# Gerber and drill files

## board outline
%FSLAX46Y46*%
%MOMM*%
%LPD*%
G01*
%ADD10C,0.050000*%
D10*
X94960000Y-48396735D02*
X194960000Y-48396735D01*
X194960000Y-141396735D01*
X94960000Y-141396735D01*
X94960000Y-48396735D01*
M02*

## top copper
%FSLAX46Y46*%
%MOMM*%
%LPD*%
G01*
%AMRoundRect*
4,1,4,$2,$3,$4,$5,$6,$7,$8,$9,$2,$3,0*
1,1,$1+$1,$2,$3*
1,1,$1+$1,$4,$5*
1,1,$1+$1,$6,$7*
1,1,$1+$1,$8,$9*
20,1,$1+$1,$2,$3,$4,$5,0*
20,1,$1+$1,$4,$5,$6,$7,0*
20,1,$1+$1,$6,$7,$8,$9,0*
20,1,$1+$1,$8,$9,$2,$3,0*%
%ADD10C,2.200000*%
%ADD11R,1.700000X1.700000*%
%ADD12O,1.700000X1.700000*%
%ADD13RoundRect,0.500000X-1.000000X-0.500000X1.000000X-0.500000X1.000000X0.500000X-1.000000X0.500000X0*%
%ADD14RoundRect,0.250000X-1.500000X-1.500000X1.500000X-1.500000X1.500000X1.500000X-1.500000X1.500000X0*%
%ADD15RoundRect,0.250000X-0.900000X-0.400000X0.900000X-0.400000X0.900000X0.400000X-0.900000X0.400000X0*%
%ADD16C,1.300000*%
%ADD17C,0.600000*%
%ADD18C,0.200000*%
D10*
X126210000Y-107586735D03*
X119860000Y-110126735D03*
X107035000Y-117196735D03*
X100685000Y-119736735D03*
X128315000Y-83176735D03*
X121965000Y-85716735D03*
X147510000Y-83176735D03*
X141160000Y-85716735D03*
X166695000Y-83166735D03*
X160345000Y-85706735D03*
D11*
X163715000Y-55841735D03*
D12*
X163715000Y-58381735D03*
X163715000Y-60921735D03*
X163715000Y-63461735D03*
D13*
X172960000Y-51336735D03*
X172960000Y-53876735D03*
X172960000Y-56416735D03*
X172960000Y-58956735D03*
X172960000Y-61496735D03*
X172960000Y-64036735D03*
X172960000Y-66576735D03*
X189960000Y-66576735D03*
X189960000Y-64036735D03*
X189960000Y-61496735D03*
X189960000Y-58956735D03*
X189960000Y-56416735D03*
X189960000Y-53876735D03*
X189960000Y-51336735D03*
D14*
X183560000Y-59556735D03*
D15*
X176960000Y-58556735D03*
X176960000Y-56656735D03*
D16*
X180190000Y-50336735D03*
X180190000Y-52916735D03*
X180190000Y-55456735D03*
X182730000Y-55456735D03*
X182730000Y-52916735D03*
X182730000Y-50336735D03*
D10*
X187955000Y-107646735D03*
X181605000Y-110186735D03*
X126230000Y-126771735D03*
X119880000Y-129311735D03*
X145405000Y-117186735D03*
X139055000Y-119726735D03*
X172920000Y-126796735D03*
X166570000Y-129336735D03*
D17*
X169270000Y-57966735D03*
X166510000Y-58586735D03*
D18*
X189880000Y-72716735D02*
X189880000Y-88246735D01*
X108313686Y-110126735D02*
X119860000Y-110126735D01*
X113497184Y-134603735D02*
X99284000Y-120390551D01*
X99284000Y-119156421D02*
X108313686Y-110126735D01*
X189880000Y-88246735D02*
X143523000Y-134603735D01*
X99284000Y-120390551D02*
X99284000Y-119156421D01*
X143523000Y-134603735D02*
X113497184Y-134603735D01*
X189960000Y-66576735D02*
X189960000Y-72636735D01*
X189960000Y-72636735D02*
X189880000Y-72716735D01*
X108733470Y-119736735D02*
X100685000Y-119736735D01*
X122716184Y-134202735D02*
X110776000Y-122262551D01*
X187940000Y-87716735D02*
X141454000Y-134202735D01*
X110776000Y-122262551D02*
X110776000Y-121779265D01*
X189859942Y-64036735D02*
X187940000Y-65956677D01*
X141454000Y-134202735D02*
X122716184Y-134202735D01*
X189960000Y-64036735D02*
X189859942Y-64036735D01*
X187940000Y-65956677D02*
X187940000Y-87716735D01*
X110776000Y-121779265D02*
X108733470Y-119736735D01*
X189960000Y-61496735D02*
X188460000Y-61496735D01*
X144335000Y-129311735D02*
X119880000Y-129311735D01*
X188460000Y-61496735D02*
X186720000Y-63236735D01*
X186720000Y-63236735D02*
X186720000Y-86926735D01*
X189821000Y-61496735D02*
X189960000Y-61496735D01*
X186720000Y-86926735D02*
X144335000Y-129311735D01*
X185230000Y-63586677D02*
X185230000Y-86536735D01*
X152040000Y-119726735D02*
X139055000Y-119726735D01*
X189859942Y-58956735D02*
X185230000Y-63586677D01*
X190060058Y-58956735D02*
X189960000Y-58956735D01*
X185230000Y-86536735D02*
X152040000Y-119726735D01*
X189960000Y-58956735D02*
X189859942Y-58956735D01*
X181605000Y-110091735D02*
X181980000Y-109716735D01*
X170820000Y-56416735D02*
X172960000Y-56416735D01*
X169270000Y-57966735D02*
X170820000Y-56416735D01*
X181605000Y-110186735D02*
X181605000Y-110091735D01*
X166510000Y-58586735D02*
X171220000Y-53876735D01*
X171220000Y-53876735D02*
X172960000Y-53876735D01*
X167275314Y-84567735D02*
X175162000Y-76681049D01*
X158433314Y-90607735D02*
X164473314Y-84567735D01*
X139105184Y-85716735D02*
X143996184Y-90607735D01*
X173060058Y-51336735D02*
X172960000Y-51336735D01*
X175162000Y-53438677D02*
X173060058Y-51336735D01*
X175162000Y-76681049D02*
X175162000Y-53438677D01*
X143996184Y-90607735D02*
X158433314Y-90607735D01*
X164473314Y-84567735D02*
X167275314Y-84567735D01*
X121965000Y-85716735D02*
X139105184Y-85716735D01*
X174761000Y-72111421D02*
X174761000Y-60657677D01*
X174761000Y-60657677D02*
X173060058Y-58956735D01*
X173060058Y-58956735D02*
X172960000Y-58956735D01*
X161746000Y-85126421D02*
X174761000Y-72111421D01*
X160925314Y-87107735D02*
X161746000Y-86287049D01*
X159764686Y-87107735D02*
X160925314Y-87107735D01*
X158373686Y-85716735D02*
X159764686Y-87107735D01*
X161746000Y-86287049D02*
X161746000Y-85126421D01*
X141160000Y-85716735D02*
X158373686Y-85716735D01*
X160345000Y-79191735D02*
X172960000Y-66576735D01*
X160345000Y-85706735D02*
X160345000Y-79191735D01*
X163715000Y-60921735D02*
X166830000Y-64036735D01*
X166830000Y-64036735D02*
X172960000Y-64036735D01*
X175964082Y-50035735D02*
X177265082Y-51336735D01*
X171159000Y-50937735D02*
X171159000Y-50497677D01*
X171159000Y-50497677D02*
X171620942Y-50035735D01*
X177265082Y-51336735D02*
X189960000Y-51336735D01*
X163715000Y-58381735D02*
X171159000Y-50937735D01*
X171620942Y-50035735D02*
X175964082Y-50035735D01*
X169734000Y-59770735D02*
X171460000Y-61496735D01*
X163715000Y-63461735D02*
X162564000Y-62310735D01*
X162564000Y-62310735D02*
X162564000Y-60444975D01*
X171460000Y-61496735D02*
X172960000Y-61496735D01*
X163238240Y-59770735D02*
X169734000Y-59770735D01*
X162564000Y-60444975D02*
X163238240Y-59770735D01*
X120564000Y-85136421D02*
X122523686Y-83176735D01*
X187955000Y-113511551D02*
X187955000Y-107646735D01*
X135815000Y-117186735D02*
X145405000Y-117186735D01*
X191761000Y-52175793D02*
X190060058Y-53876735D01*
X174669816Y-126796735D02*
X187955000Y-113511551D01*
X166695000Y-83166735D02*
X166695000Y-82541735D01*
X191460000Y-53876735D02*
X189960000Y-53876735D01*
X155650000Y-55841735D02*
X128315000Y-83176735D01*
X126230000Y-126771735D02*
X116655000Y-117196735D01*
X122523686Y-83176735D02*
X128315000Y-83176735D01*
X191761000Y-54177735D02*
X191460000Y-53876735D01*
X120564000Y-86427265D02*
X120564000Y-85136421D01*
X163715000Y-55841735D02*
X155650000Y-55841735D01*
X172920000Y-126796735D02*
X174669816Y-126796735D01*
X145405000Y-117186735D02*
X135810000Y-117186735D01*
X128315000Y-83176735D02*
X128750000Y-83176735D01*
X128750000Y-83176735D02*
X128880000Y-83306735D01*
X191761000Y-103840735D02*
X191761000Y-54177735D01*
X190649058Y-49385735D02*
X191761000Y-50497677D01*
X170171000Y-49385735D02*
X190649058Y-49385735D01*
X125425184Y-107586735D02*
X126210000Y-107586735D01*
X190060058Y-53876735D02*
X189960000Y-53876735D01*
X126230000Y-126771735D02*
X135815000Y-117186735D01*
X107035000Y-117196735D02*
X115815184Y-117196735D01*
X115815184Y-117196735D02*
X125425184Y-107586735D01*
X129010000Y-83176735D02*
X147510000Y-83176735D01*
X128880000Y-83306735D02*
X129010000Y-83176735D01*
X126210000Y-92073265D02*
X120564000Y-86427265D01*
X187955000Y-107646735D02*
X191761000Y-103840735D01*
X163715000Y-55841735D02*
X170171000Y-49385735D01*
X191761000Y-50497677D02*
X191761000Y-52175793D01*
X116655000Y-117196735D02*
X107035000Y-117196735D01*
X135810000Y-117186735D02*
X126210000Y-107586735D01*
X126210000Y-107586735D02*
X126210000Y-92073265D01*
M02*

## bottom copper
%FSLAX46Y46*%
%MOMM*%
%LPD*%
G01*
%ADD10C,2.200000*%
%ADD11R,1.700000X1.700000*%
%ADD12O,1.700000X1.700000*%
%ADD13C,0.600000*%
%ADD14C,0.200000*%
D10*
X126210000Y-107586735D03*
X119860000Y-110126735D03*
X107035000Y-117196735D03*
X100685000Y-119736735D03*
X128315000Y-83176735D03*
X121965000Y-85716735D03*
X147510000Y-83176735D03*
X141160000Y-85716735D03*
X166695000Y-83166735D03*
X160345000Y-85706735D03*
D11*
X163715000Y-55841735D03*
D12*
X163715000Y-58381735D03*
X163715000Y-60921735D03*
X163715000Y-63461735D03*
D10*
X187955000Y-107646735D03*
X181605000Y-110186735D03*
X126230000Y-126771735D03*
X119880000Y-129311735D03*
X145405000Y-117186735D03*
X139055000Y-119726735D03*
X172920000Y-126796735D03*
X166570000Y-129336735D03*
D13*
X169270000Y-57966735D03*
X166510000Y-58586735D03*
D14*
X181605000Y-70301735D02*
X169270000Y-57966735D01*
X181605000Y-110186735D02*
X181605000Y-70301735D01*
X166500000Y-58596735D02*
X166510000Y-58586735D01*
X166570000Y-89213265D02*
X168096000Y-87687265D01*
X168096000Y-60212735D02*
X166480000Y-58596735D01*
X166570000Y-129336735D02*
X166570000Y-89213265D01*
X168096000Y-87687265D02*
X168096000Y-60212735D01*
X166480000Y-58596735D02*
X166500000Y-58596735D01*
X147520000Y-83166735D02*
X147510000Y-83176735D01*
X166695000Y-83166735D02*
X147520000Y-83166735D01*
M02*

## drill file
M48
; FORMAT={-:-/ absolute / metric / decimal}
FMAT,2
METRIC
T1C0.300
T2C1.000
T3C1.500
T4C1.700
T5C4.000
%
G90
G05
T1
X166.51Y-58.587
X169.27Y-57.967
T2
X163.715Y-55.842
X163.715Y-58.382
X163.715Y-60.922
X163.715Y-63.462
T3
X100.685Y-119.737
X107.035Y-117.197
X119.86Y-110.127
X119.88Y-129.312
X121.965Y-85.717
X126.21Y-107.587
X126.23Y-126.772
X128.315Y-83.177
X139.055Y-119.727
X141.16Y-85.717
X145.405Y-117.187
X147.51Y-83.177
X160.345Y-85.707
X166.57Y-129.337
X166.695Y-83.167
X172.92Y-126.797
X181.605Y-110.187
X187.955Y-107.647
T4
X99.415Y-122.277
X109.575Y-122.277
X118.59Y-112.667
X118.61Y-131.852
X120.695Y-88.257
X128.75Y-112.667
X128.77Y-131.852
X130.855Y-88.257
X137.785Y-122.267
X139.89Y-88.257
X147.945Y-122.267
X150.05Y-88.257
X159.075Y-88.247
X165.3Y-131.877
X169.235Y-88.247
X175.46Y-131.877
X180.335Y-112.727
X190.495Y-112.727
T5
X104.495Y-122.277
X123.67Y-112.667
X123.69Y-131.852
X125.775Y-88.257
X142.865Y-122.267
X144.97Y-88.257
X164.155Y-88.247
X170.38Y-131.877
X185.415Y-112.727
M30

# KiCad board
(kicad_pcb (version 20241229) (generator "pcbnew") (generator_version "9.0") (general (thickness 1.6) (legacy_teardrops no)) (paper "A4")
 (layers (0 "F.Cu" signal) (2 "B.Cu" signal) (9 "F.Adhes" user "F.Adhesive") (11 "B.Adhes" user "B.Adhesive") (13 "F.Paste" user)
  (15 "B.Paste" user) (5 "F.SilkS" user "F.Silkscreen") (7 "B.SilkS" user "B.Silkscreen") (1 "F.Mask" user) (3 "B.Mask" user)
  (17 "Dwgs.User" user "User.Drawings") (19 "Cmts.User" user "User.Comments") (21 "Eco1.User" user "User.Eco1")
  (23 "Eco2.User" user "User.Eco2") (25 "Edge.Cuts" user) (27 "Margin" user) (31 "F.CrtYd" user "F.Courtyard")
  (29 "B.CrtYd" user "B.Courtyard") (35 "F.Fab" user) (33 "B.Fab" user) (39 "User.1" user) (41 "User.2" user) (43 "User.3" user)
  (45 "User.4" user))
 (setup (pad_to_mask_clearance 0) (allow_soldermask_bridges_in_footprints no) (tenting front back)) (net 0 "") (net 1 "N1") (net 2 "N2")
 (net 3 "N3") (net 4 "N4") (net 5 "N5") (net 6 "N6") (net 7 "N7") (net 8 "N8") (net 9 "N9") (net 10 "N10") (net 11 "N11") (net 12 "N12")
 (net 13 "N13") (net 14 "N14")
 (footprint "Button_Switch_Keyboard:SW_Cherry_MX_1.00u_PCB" (layer "F.Cu") (at 126.21 107.586735)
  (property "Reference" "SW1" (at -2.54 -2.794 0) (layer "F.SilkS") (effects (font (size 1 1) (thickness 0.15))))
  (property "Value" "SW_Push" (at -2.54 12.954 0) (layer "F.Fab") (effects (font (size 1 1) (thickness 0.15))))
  (pad "" np_thru_hole circle (at -7.62 5.08) (size 1.7 1.7) (drill 1.7) (layers "*.Cu" "*.Mask"))
  (pad "" np_thru_hole circle (at -2.54 5.08) (size 4 4) (drill 4) (layers "*.Cu" "*.Mask"))
  (pad "" np_thru_hole circle (at 2.54 5.08) (size 1.7 1.7) (drill 1.7) (layers "*.Cu" "*.Mask"))
  (pad "1" thru_hole circle (at 0 0) (size 2.2 2.2) (drill 1.5) (layers "*.Cu" "*.Mask") (remove_unused_layers no) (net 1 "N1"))
  (pad "2" thru_hole circle (at -6.35 2.54) (size 2.2 2.2) (drill 1.5) (layers "*.Cu" "*.Mask") (remove_unused_layers no) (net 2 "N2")))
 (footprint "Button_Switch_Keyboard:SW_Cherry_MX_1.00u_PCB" (layer "F.Cu") (at 107.035 117.196735)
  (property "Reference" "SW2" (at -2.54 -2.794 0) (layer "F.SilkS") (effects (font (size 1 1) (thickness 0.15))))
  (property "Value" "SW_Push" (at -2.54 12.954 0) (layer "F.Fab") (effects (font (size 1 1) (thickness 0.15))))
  (pad "" np_thru_hole circle (at -7.62 5.08) (size 1.7 1.7) (drill 1.7) (layers "*.Cu" "*.Mask"))
  (pad "" np_thru_hole circle (at -2.54 5.08) (size 4 4) (drill 4) (layers "*.Cu" "*.Mask"))
  (pad "" np_thru_hole circle (at 2.54 5.08) (size 1.7 1.7) (drill 1.7) (layers "*.Cu" "*.Mask"))
  (pad "1" thru_hole circle (at 0 0) (size 2.2 2.2) (drill 1.5) (layers "*.Cu" "*.Mask") (remove_unused_layers no) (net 1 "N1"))
  (pad "2" thru_hole circle (at -6.35 2.54) (size 2.2 2.2) (drill 1.5) (layers "*.Cu" "*.Mask") (remove_unused_layers no) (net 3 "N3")))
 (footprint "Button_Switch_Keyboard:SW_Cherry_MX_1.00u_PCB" (layer "F.Cu") (at 128.315 83.176735)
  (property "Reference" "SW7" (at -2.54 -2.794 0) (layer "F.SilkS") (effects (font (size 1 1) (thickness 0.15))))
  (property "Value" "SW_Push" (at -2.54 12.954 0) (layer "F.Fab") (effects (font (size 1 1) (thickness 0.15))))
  (pad "" np_thru_hole circle (at -7.62 5.08) (size 1.7 1.7) (drill 1.7) (layers "*.Cu" "*.Mask"))
  (pad "" np_thru_hole circle (at -2.54 5.08) (size 4 4) (drill 4) (layers "*.Cu" "*.Mask"))
  (pad "" np_thru_hole circle (at 2.54 5.08) (size 1.7 1.7) (drill 1.7) (layers "*.Cu" "*.Mask"))
  (pad "1" thru_hole circle (at 0 0) (size 2.2 2.2) (drill 1.5) (layers "*.Cu" "*.Mask") (remove_unused_layers no) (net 1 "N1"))
  (pad "2" thru_hole circle (at -6.35 2.54) (size 2.2 2.2) (drill 1.5) (layers "*.Cu" "*.Mask") (remove_unused_layers no) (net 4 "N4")))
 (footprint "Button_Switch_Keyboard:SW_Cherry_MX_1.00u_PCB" (layer "F.Cu") (at 147.51 83.176735)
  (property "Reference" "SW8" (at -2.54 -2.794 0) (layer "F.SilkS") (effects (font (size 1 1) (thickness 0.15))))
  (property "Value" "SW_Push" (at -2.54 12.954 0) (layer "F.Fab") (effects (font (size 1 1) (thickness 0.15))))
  (pad "" np_thru_hole circle (at -7.62 5.08) (size 1.7 1.7) (drill 1.7) (layers "*.Cu" "*.Mask"))
  (pad "" np_thru_hole circle (at -2.54 5.08) (size 4 4) (drill 4) (layers "*.Cu" "*.Mask"))
  (pad "" np_thru_hole circle (at 2.54 5.08) (size 1.7 1.7) (drill 1.7) (layers "*.Cu" "*.Mask"))
  (pad "1" thru_hole circle (at 0 0) (size 2.2 2.2) (drill 1.5) (layers "*.Cu" "*.Mask") (remove_unused_layers no) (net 1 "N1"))
  (pad "2" thru_hole circle (at -6.35 2.54) (size 2.2 2.2) (drill 1.5) (layers "*.Cu" "*.Mask") (remove_unused_layers no) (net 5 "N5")))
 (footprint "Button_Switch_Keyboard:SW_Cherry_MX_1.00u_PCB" (layer "F.Cu") (at 166.695 83.166735)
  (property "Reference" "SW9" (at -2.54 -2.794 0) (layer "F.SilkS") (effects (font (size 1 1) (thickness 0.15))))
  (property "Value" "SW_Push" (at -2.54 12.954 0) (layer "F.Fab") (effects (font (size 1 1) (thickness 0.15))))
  (pad "" np_thru_hole circle (at -7.62 5.08) (size 1.7 1.7) (drill 1.7) (layers "*.Cu" "*.Mask"))
  (pad "" np_thru_hole circle (at -2.54 5.08) (size 4 4) (drill 4) (layers "*.Cu" "*.Mask"))
  (pad "" np_thru_hole circle (at 2.54 5.08) (size 1.7 1.7) (drill 1.7) (layers "*.Cu" "*.Mask"))
  (pad "1" thru_hole circle (at 0 0) (size 2.2 2.2) (drill 1.5) (layers "*.Cu" "*.Mask") (remove_unused_layers no) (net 1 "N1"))
  (pad "2" thru_hole circle (at -6.35 2.54) (size 2.2 2.2) (drill 1.5) (layers "*.Cu" "*.Mask") (remove_unused_layers no) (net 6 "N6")))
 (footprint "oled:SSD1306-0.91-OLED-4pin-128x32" (layer "F.Cu") (at 127.215 53.651735)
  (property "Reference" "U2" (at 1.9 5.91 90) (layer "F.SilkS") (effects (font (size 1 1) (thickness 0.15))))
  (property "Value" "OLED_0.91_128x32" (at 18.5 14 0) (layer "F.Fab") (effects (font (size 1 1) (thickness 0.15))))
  (pad "1" thru_hole rect (at 36.5 2.19) (size 1.7 1.7) (drill 1) (layers "*.Cu" "*.Mask") (remove_unused_layers no) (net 1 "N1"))
  (pad "2" thru_hole oval (at 36.5 4.73) (size 1.7 1.7) (drill 1) (layers "*.Cu" "*.Mask") (remove_unused_layers no) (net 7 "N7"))
  (pad "3" thru_hole oval (at 36.5 7.27) (size 1.7 1.7) (drill 1) (layers "*.Cu" "*.Mask") (remove_unused_layers no) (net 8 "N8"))
  (pad "4" thru_hole oval (at 36.5 9.81) (size 1.7 1.7) (drill 1) (layers "*.Cu" "*.Mask") (remove_unused_layers no) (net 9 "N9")))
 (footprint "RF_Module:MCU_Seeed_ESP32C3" (layer "F.Cu") (at 181.46 58.956735)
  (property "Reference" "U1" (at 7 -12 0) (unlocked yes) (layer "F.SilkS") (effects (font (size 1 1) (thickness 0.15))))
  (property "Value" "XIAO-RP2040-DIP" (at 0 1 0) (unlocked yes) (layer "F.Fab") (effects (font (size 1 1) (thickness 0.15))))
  (pad "" smd roundrect (at 1.1 -0.4) (size 1.5 1.5) (layers "F.Paste") (roundrect_rratio 0.1666666667))
  (pad "" smd roundrect (at 1.1 1.6) (size 1.5 1.5) (layers "F.Paste") (roundrect_rratio 0.1666666667))
  (pad "" smd roundrect (at 3.1 -0.4) (size 1.5 1.5) (layers "F.Paste") (roundrect_rratio 0.1666666667))
  (pad "" smd roundrect (at 3.1 1.6) (size 1.5 1.5) (layers "F.Paste") (roundrect_rratio 0.1666666667))
  (pad "1" smd roundrect (at -8.5 -7.62) (size 3 2) (layers "F.Cu" "F.Mask" "F.Paste") (roundrect_rratio 0.25) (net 4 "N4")
   (thermal_bridge_angle 45))
  (pad "2" smd roundrect (at -8.5 -5.08) (size 3 2) (layers "F.Cu" "F.Mask" "F.Paste") (roundrect_rratio 0.25) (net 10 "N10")
   (thermal_bridge_angle 45))
  (pad "3" smd roundrect (at -8.5 -2.54) (size 3 2) (layers "F.Cu" "F.Mask" "F.Paste") (roundrect_rratio 0.25) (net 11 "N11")
   (thermal_bridge_angle 45))
  (pad "4" smd roundrect (at -8.5 0) (size 3 2) (layers "F.Cu" "F.Mask" "F.Paste") (roundrect_rratio 0.25) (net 5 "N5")
   (thermal_bridge_angle 45))
  (pad "5" smd roundrect (at -8.5 2.54) (size 3 2) (layers "F.Cu" "F.Mask" "F.Paste") (roundrect_rratio 0.25) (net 9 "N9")
   (thermal_bridge_angle 45))
  (pad "6" smd roundrect (at -8.5 5.08) (size 3 2) (layers "F.Cu" "F.Mask" "F.Paste") (roundrect_rratio 0.25) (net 8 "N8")
   (thermal_bridge_angle 45))
  (pad "7" smd roundrect (at -8.5 7.62) (size 3 2) (layers "F.Cu" "F.Mask" "F.Paste") (roundrect_rratio 0.25) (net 6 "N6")
   (thermal_bridge_angle 45))
  (pad "8" smd roundrect (at 8.5 7.62) (size 3 2) (layers "F.Cu" "F.Mask" "F.Paste") (roundrect_rratio 0.25) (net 2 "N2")
   (thermal_bridge_angle 45))
  (pad "9" smd roundrect (at 8.5 5.08) (size 3 2) (layers "F.Cu" "F.Mask" "F.Paste") (roundrect_rratio 0.25) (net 3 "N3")
   (thermal_bridge_angle 45))
  (pad "10" smd roundrect (at 8.5 2.54) (size 3 2) (layers "F.Cu" "F.Mask" "F.Paste") (roundrect_rratio 0.25) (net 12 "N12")
   (thermal_bridge_angle 45))
  (pad "11" smd roundrect (at 8.5 0) (size 3 2) (layers "F.Cu" "F.Mask" "F.Paste") (roundrect_rratio 0.25) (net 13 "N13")
   (thermal_bridge_angle 45))
  (pad "12" smd roundrect (at 8.5 -2.54) (size 3 2) (layers "F.Cu" "F.Mask" "F.Paste") (roundrect_rratio 0.25) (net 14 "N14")
   (thermal_bridge_angle 45))
  (pad "13" smd roundrect (at 8.5 -5.08) (size 3 2) (layers "F.Cu" "F.Mask" "F.Paste") (roundrect_rratio 0.25) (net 1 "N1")
   (thermal_bridge_angle 45))
  (pad "14" smd roundrect (at 8.5 -7.62) (size 3 2) (layers "F.Cu" "F.Mask" "F.Paste") (roundrect_rratio 0.25) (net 7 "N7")
   (thermal_bridge_angle 45))
  (pad "15" smd roundrect (at 2.1 0.6) (size 3.5 3.5) (layers "F.Cu" "F.Mask") (roundrect_rratio 0.07142857143))
  (pad "16" smd roundrect (at -4.5 -0.4) (size 2.3 1.3) (layers "F.Cu" "F.Mask" "F.Paste") (roundrect_rratio 0.1923076923))
  (pad "17" smd roundrect (at -4.5 -2.3) (size 2.3 1.3) (layers "F.Cu" "F.Mask" "F.Paste") (roundrect_rratio 0.1923076923))
  (pad "18" smd circle (at -1.27 -8.62) (size 1.3 1.3) (layers "F.Cu" "F.Mask" "F.Paste"))
  (pad "19" smd circle (at -1.27 -6.04) (size 1.3 1.3) (layers "F.Cu" "F.Mask" "F.Paste"))
  (pad "20" smd circle (at -1.27 -3.5) (size 1.3 1.3) (layers "F.Cu" "F.Mask" "F.Paste"))
  (pad "21" smd circle (at 1.27 -3.5) (size 1.3 1.3) (layers "F.Cu" "F.Mask" "F.Paste"))
  (pad "22" smd circle (at 1.27 -6.04) (size 1.3 1.3) (layers "F.Cu" "F.Mask" "F.Paste"))
  (pad "23" smd circle (at 1.27 -8.62) (size 1.3 1.3) (layers "F.Cu" "F.Mask" "F.Paste")))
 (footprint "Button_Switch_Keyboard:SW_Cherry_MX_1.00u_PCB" (layer "F.Cu") (at 187.955 107.646735)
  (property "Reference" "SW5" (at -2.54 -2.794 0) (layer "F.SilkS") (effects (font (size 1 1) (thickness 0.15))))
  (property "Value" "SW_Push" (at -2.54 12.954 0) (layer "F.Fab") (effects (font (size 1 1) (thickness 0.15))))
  (pad "" np_thru_hole circle (at -7.62 5.08) (size 1.7 1.7) (drill 1.7) (layers "*.Cu" "*.Mask"))
  (pad "" np_thru_hole circle (at -2.54 5.08) (size 4 4) (drill 4) (layers "*.Cu" "*.Mask"))
  (pad "" np_thru_hole circle (at 2.54 5.08) (size 1.7 1.7) (drill 1.7) (layers "*.Cu" "*.Mask"))
  (pad "1" thru_hole circle (at 0 0) (size 2.2 2.2) (drill 1.5) (layers "*.Cu" "*.Mask") (remove_unused_layers no) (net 1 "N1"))
  (pad "2" thru_hole circle (at -6.35 2.54) (size 2.2 2.2) (drill 1.5) (layers "*.Cu" "*.Mask") (remove_unused_layers no) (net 11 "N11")))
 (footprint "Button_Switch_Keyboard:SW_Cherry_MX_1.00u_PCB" (layer "F.Cu") (at 126.23 126.771735)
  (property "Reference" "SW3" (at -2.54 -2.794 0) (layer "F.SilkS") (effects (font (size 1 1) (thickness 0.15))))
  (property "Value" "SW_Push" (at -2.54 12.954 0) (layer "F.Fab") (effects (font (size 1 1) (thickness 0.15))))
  (pad "" np_thru_hole circle (at -7.62 5.08) (size 1.7 1.7) (drill 1.7) (layers "*.Cu" "*.Mask"))
  (pad "" np_thru_hole circle (at -2.54 5.08) (size 4 4) (drill 4) (layers "*.Cu" "*.Mask"))
  (pad "" np_thru_hole circle (at 2.54 5.08) (size 1.7 1.7) (drill 1.7) (layers "*.Cu" "*.Mask"))
  (pad "1" thru_hole circle (at 0 0) (size 2.2 2.2) (drill 1.5) (layers "*.Cu" "*.Mask") (remove_unused_layers no) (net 1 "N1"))
  (pad "2" thru_hole circle (at -6.35 2.54) (size 2.2 2.2) (drill 1.5) (layers "*.Cu" "*.Mask") (remove_unused_layers no) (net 12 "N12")))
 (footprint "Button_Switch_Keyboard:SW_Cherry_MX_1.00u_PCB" (layer "F.Cu") (at 145.405 117.186735)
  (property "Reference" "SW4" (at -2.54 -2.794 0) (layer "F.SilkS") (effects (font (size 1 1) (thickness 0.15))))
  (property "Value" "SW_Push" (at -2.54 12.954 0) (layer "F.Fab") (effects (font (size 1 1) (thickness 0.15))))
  (pad "" np_thru_hole circle (at -7.62 5.08) (size 1.7 1.7) (drill 1.7) (layers "*.Cu" "*.Mask"))
  (pad "" np_thru_hole circle (at -2.54 5.08) (size 4 4) (drill 4) (layers "*.Cu" "*.Mask"))
  (pad "" np_thru_hole circle (at 2.54 5.08) (size 1.7 1.7) (drill 1.7) (layers "*.Cu" "*.Mask"))
  (pad "1" thru_hole circle (at 0 0) (size 2.2 2.2) (drill 1.5) (layers "*.Cu" "*.Mask") (remove_unused_layers no) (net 1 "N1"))
  (pad "2" thru_hole circle (at -6.35 2.54) (size 2.2 2.2) (drill 1.5) (layers "*.Cu" "*.Mask") (remove_unused_layers no) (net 13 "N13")))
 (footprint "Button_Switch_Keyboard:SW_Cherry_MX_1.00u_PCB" (layer "F.Cu") (at 172.92 126.796735)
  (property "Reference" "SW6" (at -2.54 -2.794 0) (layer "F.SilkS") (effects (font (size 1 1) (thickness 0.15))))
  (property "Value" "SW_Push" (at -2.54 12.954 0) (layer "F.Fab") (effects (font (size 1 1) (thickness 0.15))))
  (pad "" np_thru_hole circle (at -7.62 5.08) (size 1.7 1.7) (drill 1.7) (layers "*.Cu" "*.Mask"))
  (pad "" np_thru_hole circle (at -2.54 5.08) (size 4 4) (drill 4) (layers "*.Cu" "*.Mask"))
  (pad "" np_thru_hole circle (at 2.54 5.08) (size 1.7 1.7) (drill 1.7) (layers "*.Cu" "*.Mask"))
  (pad "1" thru_hole circle (at 0 0) (size 2.2 2.2) (drill 1.5) (layers "*.Cu" "*.Mask") (remove_unused_layers no) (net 1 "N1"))
  (pad "2" thru_hole circle (at -6.35 2.54) (size 2.2 2.2) (drill 1.5) (layers "*.Cu" "*.Mask") (remove_unused_layers no) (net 10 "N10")))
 (gr_rect (start 94.96 48.396735) (end 194.96 141.396735) (stroke (width 0.05) (type default)) (fill no) (layer "Edge.Cuts"))
 (segment (start 189.88 72.716735) (end 189.88 88.246735) (width 0.2) (layer "F.Cu") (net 2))
 (segment (start 108.313686 110.126735) (end 119.86 110.126735) (width 0.2) (layer "F.Cu") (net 2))
 (segment (start 113.497184 134.603735) (end 99.284 120.390551) (width 0.2) (layer "F.Cu") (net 2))
 (segment (start 99.284 119.156421) (end 108.313686 110.126735) (width 0.2) (layer "F.Cu") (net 2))
 (segment (start 189.88 88.246735) (end 143.523 134.603735) (width 0.2) (layer "F.Cu") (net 2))
 (segment (start 99.284 120.390551) (end 99.284 119.156421) (width 0.2) (layer "F.Cu") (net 2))
 (segment (start 143.523 134.603735) (end 113.497184 134.603735) (width 0.2) (layer "F.Cu") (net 2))
 (segment (start 189.96 66.576735) (end 189.96 72.636735) (width 0.2) (layer "F.Cu") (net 2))
 (segment (start 189.96 72.636735) (end 189.88 72.716735) (width 0.2) (layer "F.Cu") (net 2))
 (segment (start 108.73347 119.736735) (end 100.685 119.736735) (width 0.2) (layer "F.Cu") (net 3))
 (segment (start 122.716184 134.202735) (end 110.776 122.262551) (width 0.2) (layer "F.Cu") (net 3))
 (segment (start 187.94 87.716735) (end 141.454 134.202735) (width 0.2) (layer "F.Cu") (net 3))
 (segment (start 110.776 122.262551) (end 110.776 121.779265) (width 0.2) (layer "F.Cu") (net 3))
 (segment (start 189.859942 64.036735) (end 187.94 65.956677) (width 0.2) (layer "F.Cu") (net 3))
 (segment (start 141.454 134.202735) (end 122.716184 134.202735) (width 0.2) (layer "F.Cu") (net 3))
 (segment (start 189.96 64.036735) (end 189.859942 64.036735) (width 0.2) (layer "F.Cu") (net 3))
 (segment (start 187.94 65.956677) (end 187.94 87.716735) (width 0.2) (layer "F.Cu") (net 3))
 (segment (start 110.776 121.779265) (end 108.73347 119.736735) (width 0.2) (layer "F.Cu") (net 3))
 (segment (start 189.96 61.496735) (end 188.46 61.496735) (width 0.2) (layer "F.Cu") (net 12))
 (segment (start 144.335 129.311735) (end 119.88 129.311735) (width 0.2) (layer "F.Cu") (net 12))
 (segment (start 188.46 61.496735) (end 186.72 63.236735) (width 0.2) (layer "F.Cu") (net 12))
 (segment (start 186.72 63.236735) (end 186.72 86.926735) (width 0.2) (layer "F.Cu") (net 12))
 (segment (start 189.821 61.496735) (end 189.96 61.496735) (width 0.2) (layer "F.Cu") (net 12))
 (segment (start 186.72 86.926735) (end 144.335 129.311735) (width 0.2) (layer "F.Cu") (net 12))
 (segment (start 185.23 63.586677) (end 185.23 86.536735) (width 0.2) (layer "F.Cu") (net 13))
 (segment (start 152.04 119.726735) (end 139.055 119.726735) (width 0.2) (layer "F.Cu") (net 13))
 (segment (start 189.859942 58.956735) (end 185.23 63.586677) (width 0.2) (layer "F.Cu") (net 13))
 (segment (start 190.060058 58.956735) (end 189.96 58.956735) (width 0.2) (layer "F.Cu") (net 13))
 (segment (start 185.23 86.536735) (end 152.04 119.726735) (width 0.2) (layer "F.Cu") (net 13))
 (segment (start 189.96 58.956735) (end 189.859942 58.956735) (width 0.2) (layer "F.Cu") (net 13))
 (segment (start 181.605 110.091735) (end 181.98 109.716735) (width 0.2) (layer "F.Cu") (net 11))
 (segment (start 170.82 56.416735) (end 172.96 56.416735) (width 0.2) (layer "F.Cu") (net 11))
 (segment (start 169.27 57.966735) (end 170.82 56.416735) (width 0.2) (layer "F.Cu") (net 11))
 (segment (start 181.605 110.186735) (end 181.605 110.091735) (width 0.2) (layer "F.Cu") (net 11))
 (via (at 169.27 57.966735) (size 0.6) (drill 0.3) (layers "F.Cu" "B.Cu") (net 11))
 (segment (start 181.605 70.301735) (end 169.27 57.966735) (width 0.2) (layer "B.Cu") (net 11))
 (segment (start 181.605 110.186735) (end 181.605 70.301735) (width 0.2) (layer "B.Cu") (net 11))
 (segment (start 166.51 58.586735) (end 171.22 53.876735) (width 0.2) (layer "F.Cu") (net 10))
 (segment (start 171.22 53.876735) (end 172.96 53.876735) (width 0.2) (layer "F.Cu") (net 10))
 (via (at 166.51 58.586735) (size 0.6) (drill 0.3) (layers "F.Cu" "B.Cu") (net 10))
 (segment (start 166.5 58.596735) (end 166.51 58.586735) (width 0.2) (layer "B.Cu") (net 10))
 (segment (start 166.57 89.213265) (end 168.096 87.687265) (width 0.2) (layer "B.Cu") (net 10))
 (segment (start 168.096 60.212735) (end 166.48 58.596735) (width 0.2) (layer "B.Cu") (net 10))
 (segment (start 166.57 129.336735) (end 166.57 89.213265) (width 0.2) (layer "B.Cu") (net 10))
 (segment (start 168.096 87.687265) (end 168.096 60.212735) (width 0.2) (layer "B.Cu") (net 10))
 (segment (start 166.48 58.596735) (end 166.5 58.596735) (width 0.2) (layer "B.Cu") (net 10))
 (segment (start 167.275314 84.567735) (end 175.162 76.681049) (width 0.2) (layer "F.Cu") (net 4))
 (segment (start 158.433314 90.607735) (end 164.473314 84.567735) (width 0.2) (layer "F.Cu") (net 4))
 (segment (start 139.105184 85.716735) (end 143.996184 90.607735) (width 0.2) (layer "F.Cu") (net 4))
 (segment (start 173.060058 51.336735) (end 172.96 51.336735) (width 0.2) (layer "F.Cu") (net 4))
 (segment (start 175.162 53.438677) (end 173.060058 51.336735) (width 0.2) (layer "F.Cu") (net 4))
 (segment (start 175.162 76.681049) (end 175.162 53.438677) (width 0.2) (layer "F.Cu") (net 4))
 (segment (start 143.996184 90.607735) (end 158.433314 90.607735) (width 0.2) (layer "F.Cu") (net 4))
 (segment (start 164.473314 84.567735) (end 167.275314 84.567735) (width 0.2) (layer "F.Cu") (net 4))
 (segment (start 121.965 85.716735) (end 139.105184 85.716735) (width 0.2) (layer "F.Cu") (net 4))
 (segment (start 174.761 72.111421) (end 174.761 60.657677) (width 0.2) (layer "F.Cu") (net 5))
 (segment (start 174.761 60.657677) (end 173.060058 58.956735) (width 0.2) (layer "F.Cu") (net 5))
 (segment (start 173.060058 58.956735) (end 172.96 58.956735) (width 0.2) (layer "F.Cu") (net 5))
 (segment (start 161.746 85.126421) (end 174.761 72.111421) (width 0.2) (layer "F.Cu") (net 5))
 (segment (start 160.925314 87.107735) (end 161.746 86.287049) (width 0.2) (layer "F.Cu") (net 5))
 (segment (start 159.764686 87.107735) (end 160.925314 87.107735) (width 0.2) (layer "F.Cu") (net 5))
 (segment (start 158.373686 85.716735) (end 159.764686 87.107735) (width 0.2) (layer "F.Cu") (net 5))
 (segment (start 161.746 86.287049) (end 161.746 85.126421) (width 0.2) (layer "F.Cu") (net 5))
 (segment (start 141.16 85.716735) (end 158.373686 85.716735) (width 0.2) (layer "F.Cu") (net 5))
 (segment (start 160.345 79.191735) (end 172.96 66.576735) (width 0.2) (layer "F.Cu") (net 6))
 (segment (start 160.345 85.706735) (end 160.345 79.191735) (width 0.2) (layer "F.Cu") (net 6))
 (segment (start 163.715 60.921735) (end 166.83 64.036735) (width 0.2) (layer "F.Cu") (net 8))
 (segment (start 166.83 64.036735) (end 172.96 64.036735) (width 0.2) (layer "F.Cu") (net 8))
 (segment (start 175.964082 50.035735) (end 177.265082 51.336735) (width 0.2) (layer "F.Cu") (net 7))
 (segment (start 171.159 50.937735) (end 171.159 50.497677) (width 0.2) (layer "F.Cu") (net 7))
 (segment (start 171.159 50.497677) (end 171.620942 50.035735) (width 0.2) (layer "F.Cu") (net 7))
 (segment (start 177.265082 51.336735) (end 189.96 51.336735) (width 0.2) (layer "F.Cu") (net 7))
 (segment (start 163.715 58.381735) (end 171.159 50.937735) (width 0.2) (layer "F.Cu") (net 7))
 (segment (start 171.620942 50.035735) (end 175.964082 50.035735) (width 0.2) (layer "F.Cu") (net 7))
 (segment (start 169.734 59.770735) (end 171.46 61.496735) (width 0.2) (layer "F.Cu") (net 9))
 (segment (start 163.715 63.461735) (end 162.564 62.310735) (width 0.2) (layer "F.Cu") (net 9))
 (segment (start 162.564 62.310735) (end 162.564 60.444975) (width 0.2) (layer "F.Cu") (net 9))
 (segment (start 171.46 61.496735) (end 172.96 61.496735) (width 0.2) (layer "F.Cu") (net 9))
 (segment (start 163.23824 59.770735) (end 169.734 59.770735) (width 0.2) (layer "F.Cu") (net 9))
 (segment (start 162.564 60.444975) (end 163.23824 59.770735) (width 0.2) (layer "F.Cu") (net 9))
 (segment (start 120.564 85.136421) (end 122.523686 83.176735) (width 0.2) (layer "F.Cu") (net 1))
 (segment (start 187.955 113.511551) (end 187.955 107.646735) (width 0.2) (layer "F.Cu") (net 1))
 (segment (start 135.815 117.186735) (end 145.405 117.186735) (width 0.2) (layer "F.Cu") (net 1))
 (segment (start 191.761 52.175793) (end 190.060058 53.876735) (width 0.2) (layer "F.Cu") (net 1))
 (segment (start 174.669816 126.796735) (end 187.955 113.511551) (width 0.2) (layer "F.Cu") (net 1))
 (segment (start 166.695 83.166735) (end 166.695 82.541735) (width 0.2) (layer "F.Cu") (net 1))
 (segment (start 191.46 53.876735) (end 189.96 53.876735) (width 0.2) (layer "F.Cu") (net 1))
 (segment (start 155.65 55.841735) (end 128.315 83.176735) (width 0.2) (layer "F.Cu") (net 1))
 (segment (start 126.23 126.771735) (end 116.655 117.196735) (width 0.2) (layer "F.Cu") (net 1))
 (segment (start 122.523686 83.176735) (end 128.315 83.176735) (width 0.2) (layer "F.Cu") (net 1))
 (segment (start 191.761 54.177735) (end 191.46 53.876735) (width 0.2) (layer "F.Cu") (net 1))
 (segment (start 120.564 86.427265) (end 120.564 85.136421) (width 0.2) (layer "F.Cu") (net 1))
 (segment (start 163.715 55.841735) (end 155.65 55.841735) (width 0.2) (layer "F.Cu") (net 1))
 (segment (start 172.92 126.796735) (end 174.669816 126.796735) (width 0.2) (layer "F.Cu") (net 1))
 (segment (start 145.405 117.186735) (end 135.81 117.186735) (width 0.2) (layer "F.Cu") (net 1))
 (segment (start 128.315 83.176735) (end 128.75 83.176735) (width 0.2) (layer "F.Cu") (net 1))
 (segment (start 128.75 83.176735) (end 128.88 83.306735) (width 0.2) (layer "F.Cu") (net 1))
 (segment (start 191.761 103.840735) (end 191.761 54.177735) (width 0.2) (layer "F.Cu") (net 1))
 (segment (start 190.649058 49.385735) (end 191.761 50.497677) (width 0.2) (layer "F.Cu") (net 1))
 (segment (start 170.171 49.385735) (end 190.649058 49.385735) (width 0.2) (layer "F.Cu") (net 1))
 (segment (start 125.425184 107.586735) (end 126.21 107.586735) (width 0.2) (layer "F.Cu") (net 1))
 (segment (start 190.060058 53.876735) (end 189.96 53.876735) (width 0.2) (layer "F.Cu") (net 1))
 (segment (start 126.23 126.771735) (end 135.815 117.186735) (width 0.2) (layer "F.Cu") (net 1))
 (segment (start 107.035 117.196735) (end 115.815184 117.196735) (width 0.2) (layer "F.Cu") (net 1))
 (segment (start 115.815184 117.196735) (end 125.425184 107.586735) (width 0.2) (layer "F.Cu") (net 1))
 (segment (start 129.01 83.176735) (end 147.51 83.176735) (width 0.2) (layer "F.Cu") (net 1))
 (segment (start 128.88 83.306735) (end 129.01 83.176735) (width 0.2) (layer "F.Cu") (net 1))
 (segment (start 126.21 92.073265) (end 120.564 86.427265) (width 0.2) (layer "F.Cu") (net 1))
 (segment (start 187.955 107.646735) (end 191.761 103.840735) (width 0.2) (layer "F.Cu") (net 1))
 (segment (start 163.715 55.841735) (end 170.171 49.385735) (width 0.2) (layer "F.Cu") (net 1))
 (segment (start 191.761 50.497677) (end 191.761 52.175793) (width 0.2) (layer "F.Cu") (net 1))
 (segment (start 116.655 117.196735) (end 107.035 117.196735) (width 0.2) (layer "F.Cu") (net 1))
 (segment (start 135.81 117.186735) (end 126.21 107.586735) (width 0.2) (layer "F.Cu") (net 1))
 (segment (start 126.21 107.586735) (end 126.21 92.073265) (width 0.2) (layer "F.Cu") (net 1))
 (segment (start 147.52 83.166735) (end 147.51 83.176735) (width 0.2) (layer "B.Cu") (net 1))
 (segment (start 166.695 83.166735) (end 147.52 83.166735) (width 0.2) (layer "B.Cu") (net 1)))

